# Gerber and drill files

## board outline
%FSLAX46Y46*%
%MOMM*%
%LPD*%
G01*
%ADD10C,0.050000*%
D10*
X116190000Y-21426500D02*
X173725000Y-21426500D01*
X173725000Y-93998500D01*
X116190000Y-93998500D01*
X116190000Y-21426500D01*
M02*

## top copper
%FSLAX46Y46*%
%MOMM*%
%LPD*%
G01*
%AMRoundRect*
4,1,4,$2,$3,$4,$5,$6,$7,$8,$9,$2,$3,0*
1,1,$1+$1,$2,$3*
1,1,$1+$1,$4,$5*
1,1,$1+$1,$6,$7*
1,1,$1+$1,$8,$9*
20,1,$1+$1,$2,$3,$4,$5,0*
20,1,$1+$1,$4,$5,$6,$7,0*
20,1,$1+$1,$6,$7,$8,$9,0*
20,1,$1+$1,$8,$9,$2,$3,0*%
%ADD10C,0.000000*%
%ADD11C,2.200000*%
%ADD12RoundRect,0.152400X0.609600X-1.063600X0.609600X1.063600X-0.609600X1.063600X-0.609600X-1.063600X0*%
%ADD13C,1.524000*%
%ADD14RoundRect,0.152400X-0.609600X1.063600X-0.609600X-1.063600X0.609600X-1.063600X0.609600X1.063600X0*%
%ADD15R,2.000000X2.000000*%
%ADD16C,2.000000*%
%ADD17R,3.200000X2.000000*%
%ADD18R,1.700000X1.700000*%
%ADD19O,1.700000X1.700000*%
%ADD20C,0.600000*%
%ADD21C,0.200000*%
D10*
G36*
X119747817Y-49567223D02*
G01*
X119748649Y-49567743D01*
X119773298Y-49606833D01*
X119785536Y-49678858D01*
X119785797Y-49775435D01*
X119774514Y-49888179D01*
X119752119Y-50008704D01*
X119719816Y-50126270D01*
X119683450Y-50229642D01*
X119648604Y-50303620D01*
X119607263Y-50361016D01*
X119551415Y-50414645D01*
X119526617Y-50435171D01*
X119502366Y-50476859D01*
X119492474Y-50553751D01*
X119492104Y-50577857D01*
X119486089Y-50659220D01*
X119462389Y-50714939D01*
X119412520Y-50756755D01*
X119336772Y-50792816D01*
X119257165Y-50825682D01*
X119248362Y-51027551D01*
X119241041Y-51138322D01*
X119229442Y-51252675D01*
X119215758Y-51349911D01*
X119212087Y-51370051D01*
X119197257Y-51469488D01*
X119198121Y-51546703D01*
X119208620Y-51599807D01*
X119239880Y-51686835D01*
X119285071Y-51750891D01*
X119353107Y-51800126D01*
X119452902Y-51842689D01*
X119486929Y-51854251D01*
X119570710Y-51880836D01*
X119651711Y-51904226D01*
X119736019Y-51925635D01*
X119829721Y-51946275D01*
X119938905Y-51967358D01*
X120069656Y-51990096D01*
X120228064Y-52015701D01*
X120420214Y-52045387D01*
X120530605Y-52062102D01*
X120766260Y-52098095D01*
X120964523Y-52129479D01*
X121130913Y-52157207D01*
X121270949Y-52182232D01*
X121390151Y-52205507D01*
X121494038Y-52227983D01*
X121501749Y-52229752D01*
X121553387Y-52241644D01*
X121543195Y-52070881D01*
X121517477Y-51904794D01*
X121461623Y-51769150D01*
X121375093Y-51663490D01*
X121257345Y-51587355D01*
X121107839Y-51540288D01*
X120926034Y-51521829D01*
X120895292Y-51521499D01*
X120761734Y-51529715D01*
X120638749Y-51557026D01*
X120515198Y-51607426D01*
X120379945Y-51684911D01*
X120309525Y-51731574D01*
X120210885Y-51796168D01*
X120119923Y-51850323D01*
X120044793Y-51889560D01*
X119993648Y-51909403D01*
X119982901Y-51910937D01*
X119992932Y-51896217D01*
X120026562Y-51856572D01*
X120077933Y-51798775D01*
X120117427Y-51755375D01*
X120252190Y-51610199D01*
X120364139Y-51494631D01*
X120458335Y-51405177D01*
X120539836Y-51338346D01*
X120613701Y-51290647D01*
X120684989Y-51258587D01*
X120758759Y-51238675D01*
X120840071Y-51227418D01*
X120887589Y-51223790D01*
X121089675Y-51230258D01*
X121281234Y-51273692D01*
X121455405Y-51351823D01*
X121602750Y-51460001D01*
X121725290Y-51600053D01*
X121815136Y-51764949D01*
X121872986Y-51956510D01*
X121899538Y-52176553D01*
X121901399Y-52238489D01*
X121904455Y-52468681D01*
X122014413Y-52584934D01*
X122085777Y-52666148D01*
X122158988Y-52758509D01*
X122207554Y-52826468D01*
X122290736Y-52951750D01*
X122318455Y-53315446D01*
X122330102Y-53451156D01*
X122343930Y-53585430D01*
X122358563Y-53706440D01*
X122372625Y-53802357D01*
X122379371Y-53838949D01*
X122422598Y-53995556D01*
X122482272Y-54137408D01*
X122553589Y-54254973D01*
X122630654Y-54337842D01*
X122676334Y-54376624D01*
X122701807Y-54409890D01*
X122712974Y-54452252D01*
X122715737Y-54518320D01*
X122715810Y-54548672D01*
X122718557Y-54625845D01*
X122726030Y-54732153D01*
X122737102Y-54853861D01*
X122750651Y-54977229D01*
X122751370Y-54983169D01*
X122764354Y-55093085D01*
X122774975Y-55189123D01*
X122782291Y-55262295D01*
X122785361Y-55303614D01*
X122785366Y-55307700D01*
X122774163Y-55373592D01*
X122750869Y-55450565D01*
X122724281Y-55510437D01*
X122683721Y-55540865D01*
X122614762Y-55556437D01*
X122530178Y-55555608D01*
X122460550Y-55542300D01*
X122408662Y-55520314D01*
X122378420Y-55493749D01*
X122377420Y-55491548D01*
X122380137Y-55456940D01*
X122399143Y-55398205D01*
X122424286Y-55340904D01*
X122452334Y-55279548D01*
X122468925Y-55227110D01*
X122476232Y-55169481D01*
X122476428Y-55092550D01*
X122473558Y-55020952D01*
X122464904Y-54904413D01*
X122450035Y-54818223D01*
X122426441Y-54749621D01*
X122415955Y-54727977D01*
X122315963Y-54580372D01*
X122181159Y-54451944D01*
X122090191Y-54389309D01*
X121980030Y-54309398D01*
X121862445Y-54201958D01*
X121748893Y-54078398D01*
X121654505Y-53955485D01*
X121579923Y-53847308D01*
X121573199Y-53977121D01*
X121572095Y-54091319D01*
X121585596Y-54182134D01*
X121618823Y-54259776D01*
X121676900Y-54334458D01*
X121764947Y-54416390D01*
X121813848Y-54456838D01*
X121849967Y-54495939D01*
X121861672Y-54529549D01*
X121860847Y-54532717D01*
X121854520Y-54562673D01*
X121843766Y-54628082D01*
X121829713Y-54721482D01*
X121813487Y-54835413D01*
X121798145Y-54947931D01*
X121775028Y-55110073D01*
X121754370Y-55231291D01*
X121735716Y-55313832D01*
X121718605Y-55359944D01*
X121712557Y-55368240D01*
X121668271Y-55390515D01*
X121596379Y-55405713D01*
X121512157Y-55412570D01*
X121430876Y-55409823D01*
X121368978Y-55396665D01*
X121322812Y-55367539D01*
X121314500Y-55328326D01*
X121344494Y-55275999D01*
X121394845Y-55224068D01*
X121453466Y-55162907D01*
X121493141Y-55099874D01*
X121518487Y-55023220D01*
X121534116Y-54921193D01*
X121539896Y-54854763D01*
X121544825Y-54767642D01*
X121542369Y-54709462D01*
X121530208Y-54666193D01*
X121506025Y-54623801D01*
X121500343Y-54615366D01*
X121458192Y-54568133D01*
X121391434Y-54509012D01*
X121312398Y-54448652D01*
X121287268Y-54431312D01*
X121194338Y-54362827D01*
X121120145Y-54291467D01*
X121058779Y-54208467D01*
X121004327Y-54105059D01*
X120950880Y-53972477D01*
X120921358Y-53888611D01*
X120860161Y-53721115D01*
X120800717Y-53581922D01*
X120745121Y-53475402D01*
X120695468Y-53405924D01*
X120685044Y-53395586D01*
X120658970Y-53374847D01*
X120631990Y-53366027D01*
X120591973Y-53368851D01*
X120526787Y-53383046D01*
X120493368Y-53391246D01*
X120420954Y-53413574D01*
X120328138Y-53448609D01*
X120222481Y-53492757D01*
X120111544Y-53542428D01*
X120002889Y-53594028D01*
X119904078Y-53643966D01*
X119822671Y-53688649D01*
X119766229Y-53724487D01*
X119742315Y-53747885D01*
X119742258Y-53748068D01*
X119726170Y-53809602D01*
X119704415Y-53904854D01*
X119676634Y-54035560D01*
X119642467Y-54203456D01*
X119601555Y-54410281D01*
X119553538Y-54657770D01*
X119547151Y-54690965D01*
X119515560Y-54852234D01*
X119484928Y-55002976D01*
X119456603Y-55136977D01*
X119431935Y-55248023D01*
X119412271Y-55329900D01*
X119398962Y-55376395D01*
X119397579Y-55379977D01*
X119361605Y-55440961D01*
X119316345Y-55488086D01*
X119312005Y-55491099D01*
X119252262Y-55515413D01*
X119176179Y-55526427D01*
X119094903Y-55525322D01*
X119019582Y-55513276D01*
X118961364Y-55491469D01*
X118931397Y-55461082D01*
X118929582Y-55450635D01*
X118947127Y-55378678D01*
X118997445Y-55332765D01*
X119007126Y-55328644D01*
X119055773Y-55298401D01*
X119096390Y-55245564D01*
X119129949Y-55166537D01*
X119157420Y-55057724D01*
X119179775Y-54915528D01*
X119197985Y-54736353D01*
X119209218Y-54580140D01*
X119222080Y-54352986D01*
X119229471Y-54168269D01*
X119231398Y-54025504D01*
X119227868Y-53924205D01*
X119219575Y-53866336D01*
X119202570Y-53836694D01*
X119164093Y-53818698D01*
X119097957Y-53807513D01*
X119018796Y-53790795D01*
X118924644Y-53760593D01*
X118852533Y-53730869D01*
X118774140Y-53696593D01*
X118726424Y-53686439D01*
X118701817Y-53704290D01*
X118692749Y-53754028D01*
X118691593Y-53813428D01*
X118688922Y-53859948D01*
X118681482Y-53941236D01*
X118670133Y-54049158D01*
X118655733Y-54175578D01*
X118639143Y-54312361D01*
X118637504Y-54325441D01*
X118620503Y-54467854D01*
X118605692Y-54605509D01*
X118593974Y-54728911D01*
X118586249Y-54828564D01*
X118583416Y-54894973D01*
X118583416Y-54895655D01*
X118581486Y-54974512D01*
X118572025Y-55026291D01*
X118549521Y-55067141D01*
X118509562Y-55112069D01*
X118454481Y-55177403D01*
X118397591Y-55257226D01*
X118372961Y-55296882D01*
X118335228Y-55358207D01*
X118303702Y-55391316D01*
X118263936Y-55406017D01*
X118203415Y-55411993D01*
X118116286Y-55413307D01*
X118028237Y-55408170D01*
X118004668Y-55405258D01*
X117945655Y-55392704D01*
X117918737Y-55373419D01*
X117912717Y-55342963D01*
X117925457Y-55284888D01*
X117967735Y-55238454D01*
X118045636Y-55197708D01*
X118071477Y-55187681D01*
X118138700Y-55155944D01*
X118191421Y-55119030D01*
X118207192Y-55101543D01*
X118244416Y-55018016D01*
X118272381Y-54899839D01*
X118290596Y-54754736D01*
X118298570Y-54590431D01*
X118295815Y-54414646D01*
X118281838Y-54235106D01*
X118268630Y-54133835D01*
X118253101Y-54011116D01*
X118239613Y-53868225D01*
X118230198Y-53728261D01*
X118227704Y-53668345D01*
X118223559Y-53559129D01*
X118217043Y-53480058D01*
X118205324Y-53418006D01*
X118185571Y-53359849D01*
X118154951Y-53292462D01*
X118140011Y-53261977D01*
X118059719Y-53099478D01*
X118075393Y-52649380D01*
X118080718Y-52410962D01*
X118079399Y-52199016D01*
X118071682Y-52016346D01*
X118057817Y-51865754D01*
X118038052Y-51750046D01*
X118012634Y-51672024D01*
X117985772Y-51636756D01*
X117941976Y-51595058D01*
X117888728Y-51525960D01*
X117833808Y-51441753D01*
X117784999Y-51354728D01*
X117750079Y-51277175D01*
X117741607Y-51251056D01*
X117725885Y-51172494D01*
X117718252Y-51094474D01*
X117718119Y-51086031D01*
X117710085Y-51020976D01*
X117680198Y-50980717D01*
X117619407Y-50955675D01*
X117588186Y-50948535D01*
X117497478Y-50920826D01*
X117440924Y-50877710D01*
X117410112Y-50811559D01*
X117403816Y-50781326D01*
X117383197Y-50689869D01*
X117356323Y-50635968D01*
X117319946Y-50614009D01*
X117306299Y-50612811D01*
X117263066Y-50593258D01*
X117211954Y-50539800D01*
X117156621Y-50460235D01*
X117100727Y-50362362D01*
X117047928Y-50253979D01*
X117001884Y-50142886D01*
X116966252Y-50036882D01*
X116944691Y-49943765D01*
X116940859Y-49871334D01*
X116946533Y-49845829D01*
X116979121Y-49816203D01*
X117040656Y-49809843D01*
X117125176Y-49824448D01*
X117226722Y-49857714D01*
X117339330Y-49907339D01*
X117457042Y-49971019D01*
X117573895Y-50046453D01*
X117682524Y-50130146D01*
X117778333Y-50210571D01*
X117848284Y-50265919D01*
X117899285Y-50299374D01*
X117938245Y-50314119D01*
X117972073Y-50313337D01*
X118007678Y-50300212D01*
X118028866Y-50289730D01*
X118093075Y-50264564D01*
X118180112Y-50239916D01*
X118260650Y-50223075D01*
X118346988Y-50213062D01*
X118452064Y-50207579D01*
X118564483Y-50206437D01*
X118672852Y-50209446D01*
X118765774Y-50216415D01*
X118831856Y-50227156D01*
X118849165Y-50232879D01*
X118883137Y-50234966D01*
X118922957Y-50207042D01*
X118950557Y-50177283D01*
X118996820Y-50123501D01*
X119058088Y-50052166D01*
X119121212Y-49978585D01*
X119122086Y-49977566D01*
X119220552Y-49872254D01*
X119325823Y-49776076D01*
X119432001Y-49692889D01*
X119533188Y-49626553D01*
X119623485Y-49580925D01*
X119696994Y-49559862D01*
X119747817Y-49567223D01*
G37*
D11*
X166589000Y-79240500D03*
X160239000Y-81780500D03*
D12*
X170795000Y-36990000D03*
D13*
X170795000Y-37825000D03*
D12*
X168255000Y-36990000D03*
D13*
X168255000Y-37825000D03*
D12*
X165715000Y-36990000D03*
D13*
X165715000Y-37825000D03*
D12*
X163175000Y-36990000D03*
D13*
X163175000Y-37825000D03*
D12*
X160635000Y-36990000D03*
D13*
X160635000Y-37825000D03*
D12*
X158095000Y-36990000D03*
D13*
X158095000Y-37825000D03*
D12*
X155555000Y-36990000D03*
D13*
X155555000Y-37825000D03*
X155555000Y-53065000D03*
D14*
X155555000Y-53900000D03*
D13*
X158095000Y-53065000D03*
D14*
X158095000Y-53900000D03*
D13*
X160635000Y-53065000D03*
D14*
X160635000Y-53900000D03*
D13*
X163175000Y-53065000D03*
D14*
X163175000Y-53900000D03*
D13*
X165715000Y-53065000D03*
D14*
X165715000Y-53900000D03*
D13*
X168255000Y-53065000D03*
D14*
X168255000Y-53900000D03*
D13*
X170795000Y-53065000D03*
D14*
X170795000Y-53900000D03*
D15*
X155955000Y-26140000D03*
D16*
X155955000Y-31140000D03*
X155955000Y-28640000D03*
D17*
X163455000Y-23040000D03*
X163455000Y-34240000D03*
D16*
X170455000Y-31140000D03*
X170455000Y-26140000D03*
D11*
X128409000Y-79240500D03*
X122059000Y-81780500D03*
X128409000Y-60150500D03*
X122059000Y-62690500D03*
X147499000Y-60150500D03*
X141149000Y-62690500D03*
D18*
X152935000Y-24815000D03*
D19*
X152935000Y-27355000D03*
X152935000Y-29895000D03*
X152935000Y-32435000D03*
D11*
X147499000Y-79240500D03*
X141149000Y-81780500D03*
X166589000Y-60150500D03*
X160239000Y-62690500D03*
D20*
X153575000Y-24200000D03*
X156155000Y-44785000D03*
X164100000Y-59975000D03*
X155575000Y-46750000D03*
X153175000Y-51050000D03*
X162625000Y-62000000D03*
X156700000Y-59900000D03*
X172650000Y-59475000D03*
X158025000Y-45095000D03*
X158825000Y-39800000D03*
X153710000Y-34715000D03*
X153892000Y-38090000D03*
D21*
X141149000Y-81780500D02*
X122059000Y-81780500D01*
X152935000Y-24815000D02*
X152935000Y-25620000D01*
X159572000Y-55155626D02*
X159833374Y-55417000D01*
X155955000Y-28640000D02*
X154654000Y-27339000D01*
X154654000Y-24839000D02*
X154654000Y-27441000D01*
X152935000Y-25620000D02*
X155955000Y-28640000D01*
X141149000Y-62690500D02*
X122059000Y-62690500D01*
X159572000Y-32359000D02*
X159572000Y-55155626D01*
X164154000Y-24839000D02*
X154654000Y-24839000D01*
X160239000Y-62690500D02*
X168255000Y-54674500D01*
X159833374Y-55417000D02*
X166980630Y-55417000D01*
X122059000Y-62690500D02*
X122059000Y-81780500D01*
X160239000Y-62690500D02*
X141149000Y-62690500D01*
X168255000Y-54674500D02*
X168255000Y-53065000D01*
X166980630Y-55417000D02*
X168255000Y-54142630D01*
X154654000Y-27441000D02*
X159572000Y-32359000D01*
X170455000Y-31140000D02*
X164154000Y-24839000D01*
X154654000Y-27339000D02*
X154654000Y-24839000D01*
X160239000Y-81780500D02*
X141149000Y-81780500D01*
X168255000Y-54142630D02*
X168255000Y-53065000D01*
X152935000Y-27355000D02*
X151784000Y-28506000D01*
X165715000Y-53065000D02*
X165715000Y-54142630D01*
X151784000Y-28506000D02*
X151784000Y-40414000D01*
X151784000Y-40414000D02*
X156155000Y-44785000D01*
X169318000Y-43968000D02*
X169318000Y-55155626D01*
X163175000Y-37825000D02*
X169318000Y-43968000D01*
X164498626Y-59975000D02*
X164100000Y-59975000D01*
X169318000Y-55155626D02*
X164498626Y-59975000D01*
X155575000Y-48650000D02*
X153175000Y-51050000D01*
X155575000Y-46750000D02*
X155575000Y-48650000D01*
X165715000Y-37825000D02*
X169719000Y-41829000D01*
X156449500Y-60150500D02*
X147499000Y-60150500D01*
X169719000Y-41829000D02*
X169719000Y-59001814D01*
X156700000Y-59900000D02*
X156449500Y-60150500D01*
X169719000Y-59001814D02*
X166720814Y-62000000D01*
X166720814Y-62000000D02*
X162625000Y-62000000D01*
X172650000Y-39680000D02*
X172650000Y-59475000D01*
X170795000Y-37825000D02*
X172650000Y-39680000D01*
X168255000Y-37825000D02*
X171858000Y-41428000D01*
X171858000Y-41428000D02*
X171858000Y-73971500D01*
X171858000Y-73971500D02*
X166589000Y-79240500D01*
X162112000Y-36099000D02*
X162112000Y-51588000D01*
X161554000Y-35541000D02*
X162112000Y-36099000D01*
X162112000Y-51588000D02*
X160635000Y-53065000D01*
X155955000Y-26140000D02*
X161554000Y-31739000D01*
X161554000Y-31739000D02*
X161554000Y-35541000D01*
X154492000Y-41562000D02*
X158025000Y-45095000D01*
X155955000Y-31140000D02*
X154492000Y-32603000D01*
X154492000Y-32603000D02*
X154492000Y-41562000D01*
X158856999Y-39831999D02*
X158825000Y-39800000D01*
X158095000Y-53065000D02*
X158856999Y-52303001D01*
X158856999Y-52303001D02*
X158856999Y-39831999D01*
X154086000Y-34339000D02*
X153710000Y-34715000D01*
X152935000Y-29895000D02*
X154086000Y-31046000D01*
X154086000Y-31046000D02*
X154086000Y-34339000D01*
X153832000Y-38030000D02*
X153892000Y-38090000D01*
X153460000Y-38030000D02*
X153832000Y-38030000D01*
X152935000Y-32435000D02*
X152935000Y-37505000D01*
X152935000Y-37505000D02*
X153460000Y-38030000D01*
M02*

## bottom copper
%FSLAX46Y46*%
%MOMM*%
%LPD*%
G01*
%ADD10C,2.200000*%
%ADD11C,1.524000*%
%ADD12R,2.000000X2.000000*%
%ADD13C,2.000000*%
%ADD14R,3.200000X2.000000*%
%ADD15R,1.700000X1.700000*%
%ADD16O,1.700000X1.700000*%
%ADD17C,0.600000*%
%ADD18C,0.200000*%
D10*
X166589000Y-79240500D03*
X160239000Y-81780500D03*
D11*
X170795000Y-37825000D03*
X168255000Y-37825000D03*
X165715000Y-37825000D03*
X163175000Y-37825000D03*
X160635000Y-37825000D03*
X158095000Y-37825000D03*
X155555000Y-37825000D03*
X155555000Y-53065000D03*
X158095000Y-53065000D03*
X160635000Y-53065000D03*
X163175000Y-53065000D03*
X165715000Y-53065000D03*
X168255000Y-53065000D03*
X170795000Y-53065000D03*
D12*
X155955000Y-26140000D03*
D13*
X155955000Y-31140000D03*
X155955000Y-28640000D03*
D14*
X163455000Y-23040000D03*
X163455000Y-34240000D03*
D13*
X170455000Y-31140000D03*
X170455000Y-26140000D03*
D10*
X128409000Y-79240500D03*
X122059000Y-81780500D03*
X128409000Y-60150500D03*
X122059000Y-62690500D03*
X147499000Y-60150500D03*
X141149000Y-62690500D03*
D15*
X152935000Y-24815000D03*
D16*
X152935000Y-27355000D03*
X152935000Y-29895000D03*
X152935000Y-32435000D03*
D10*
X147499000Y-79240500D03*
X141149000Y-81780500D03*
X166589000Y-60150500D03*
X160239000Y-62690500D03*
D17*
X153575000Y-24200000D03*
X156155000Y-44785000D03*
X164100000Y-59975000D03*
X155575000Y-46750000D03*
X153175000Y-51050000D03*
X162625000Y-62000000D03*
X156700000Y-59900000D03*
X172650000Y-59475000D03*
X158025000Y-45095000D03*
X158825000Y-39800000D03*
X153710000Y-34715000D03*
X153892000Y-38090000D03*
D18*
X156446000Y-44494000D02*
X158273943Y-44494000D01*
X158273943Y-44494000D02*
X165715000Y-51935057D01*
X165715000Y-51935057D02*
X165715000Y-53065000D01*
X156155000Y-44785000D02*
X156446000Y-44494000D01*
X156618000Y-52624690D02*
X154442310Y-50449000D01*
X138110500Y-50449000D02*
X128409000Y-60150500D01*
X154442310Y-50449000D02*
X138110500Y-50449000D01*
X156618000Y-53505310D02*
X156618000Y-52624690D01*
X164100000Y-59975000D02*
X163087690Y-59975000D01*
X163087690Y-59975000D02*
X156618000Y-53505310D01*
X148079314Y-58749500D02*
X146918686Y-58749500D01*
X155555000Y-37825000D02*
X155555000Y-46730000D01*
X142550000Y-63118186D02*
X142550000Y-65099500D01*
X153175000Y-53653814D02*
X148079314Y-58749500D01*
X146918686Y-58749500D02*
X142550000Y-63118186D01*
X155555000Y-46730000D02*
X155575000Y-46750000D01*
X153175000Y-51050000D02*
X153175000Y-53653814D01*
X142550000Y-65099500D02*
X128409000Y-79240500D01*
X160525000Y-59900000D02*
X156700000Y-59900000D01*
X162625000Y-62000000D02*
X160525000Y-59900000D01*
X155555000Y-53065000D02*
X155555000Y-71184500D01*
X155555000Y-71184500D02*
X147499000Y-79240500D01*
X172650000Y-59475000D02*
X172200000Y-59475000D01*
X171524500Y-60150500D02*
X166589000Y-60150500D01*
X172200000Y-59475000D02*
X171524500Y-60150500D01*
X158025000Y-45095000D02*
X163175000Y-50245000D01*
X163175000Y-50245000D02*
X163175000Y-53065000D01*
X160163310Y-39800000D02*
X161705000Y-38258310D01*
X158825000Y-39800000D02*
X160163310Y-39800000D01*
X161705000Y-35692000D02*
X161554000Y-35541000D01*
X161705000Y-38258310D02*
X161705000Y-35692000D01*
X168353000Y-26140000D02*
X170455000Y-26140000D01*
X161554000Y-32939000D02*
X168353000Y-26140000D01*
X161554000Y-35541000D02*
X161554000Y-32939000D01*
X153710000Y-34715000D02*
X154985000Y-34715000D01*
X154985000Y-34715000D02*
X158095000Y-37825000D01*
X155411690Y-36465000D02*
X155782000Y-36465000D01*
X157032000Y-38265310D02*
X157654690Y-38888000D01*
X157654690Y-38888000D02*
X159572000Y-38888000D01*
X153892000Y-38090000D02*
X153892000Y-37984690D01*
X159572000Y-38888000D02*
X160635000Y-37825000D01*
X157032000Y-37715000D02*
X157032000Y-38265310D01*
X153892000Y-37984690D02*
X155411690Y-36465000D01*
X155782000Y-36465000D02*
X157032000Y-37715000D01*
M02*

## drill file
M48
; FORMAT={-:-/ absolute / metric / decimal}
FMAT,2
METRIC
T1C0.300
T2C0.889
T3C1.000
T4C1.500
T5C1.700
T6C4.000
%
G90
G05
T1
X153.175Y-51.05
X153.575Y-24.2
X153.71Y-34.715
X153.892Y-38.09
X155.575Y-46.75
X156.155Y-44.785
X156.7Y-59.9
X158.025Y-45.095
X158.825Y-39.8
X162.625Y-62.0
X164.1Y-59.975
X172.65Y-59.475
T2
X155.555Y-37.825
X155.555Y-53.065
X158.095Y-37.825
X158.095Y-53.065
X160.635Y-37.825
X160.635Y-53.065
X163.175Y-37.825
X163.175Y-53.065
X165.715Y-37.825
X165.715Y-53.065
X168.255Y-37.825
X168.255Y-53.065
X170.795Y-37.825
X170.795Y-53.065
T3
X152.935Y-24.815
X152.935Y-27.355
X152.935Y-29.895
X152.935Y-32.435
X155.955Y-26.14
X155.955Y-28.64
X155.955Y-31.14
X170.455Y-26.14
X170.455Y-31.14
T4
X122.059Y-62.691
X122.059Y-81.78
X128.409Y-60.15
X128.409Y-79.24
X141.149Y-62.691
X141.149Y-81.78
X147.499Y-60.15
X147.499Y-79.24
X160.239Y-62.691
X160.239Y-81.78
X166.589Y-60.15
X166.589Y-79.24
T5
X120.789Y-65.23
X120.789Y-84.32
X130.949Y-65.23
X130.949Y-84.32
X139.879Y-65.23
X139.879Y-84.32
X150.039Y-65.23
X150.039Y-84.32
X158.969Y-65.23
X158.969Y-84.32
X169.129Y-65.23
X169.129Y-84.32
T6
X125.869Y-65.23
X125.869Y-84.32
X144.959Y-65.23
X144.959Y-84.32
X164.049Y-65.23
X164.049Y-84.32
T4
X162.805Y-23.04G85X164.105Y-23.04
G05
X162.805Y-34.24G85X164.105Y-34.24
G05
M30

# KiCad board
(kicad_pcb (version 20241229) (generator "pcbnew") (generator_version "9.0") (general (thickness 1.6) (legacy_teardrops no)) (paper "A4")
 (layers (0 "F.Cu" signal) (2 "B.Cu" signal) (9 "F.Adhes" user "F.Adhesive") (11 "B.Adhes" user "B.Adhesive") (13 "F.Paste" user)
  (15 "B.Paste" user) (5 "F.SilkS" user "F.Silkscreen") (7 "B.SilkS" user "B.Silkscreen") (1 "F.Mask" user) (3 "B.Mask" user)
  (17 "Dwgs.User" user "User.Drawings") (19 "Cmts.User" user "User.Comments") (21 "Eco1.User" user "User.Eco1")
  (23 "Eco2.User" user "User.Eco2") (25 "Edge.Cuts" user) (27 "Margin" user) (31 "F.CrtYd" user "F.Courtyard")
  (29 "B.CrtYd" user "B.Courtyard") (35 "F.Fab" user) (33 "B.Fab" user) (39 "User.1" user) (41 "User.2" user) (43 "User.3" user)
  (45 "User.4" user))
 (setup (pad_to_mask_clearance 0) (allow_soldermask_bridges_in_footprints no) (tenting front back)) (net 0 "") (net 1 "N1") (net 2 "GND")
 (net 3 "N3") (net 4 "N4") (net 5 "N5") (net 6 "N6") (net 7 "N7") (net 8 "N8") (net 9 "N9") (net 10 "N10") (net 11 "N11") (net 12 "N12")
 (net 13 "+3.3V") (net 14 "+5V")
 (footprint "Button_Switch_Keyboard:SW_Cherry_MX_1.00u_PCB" (layer "F.Cu") (at 166.589 79.2405)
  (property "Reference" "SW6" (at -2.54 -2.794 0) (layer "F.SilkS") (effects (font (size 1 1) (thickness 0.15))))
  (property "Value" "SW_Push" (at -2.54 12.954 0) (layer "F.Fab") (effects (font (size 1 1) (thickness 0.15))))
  (pad "" np_thru_hole circle (at -7.62 5.08) (size 1.7 1.7) (drill 1.7) (layers "*.Cu" "*.Mask"))
  (pad "" np_thru_hole circle (at -2.54 5.08) (size 4 4) (drill 4) (layers "*.Cu" "*.Mask"))
  (pad "" np_thru_hole circle (at 2.54 5.08) (size 1.7 1.7) (drill 1.7) (layers "*.Cu" "*.Mask"))
  (pad "1" thru_hole circle (at 0 0) (size 2.2 2.2) (drill 1.5) (layers "*.Cu" "*.Mask") (remove_unused_layers no) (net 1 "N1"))
  (pad "2" thru_hole circle (at -6.35 2.54) (size 2.2 2.2) (drill 1.5) (layers "*.Cu" "*.Mask") (remove_unused_layers no) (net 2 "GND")))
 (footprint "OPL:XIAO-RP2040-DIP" (layer "F.Cu") (at 163.175 45.445 -90)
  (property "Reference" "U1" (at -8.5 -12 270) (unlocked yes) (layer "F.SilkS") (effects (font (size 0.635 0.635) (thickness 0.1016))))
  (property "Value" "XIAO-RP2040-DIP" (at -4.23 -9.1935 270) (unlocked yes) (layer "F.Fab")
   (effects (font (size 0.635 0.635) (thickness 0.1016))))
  (pad "1" smd roundrect (at -8.455 -7.62 90) (size 2.432 1.524) (layers "F.Cu" "F.Mask") (roundrect_rratio 0.1) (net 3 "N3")
   (thermal_bridge_angle 45))
  (pad "1" thru_hole circle (at -7.62 -7.62 90) (size 1.524 1.524) (drill 0.889) (layers "*.Cu" "*.Mask") (remove_unused_layers no)
   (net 3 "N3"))
  (pad "2" smd roundrect (at -8.455 -5.08 90) (size 2.432 1.524) (layers "F.Cu" "F.Mask") (roundrect_rratio 0.1) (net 1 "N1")
   (thermal_bridge_angle 45))
  (pad "2" thru_hole circle (at -7.62 -5.08 90) (size 1.524 1.524) (drill 0.889) (layers "*.Cu" "*.Mask") (remove_unused_layers no)
   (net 1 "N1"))
  (pad "3" smd roundrect (at -8.455 -2.54 90) (size 2.432 1.524) (layers "F.Cu" "F.Mask") (roundrect_rratio 0.1) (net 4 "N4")
   (thermal_bridge_angle 45))
  (pad "3" thru_hole circle (at -7.62 -2.54 90) (size 1.524 1.524) (drill 0.889) (layers "*.Cu" "*.Mask") (remove_unused_layers no)
   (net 4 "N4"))
  (pad "4" smd roundrect (at -8.455 0 90) (size 2.432 1.524) (layers "F.Cu" "F.Mask") (roundrect_rratio 0.1) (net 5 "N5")
   (thermal_bridge_angle 45))
  (pad "4" thru_hole circle (at -7.62 0 90) (size 1.524 1.524) (drill 0.889) (layers "*.Cu" "*.Mask") (remove_unused_layers no) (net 5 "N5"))
  (pad "5" smd roundrect (at -8.455 2.54 90) (size 2.432 1.524) (layers "F.Cu" "F.Mask") (roundrect_rratio 0.1) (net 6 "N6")
   (thermal_bridge_angle 45))
  (pad "5" thru_hole circle (at -7.62 2.54 90) (size 1.524 1.524) (drill 0.889) (layers "*.Cu" "*.Mask") (remove_unused_layers no)
   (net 6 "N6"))
  (pad "6" smd roundrect (at -8.455 5.08 90) (size 2.432 1.524) (layers "F.Cu" "F.Mask") (roundrect_rratio 0.1) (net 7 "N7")
   (thermal_bridge_angle 45))
  (pad "6" thru_hole circle (at -7.62 5.08 90) (size 1.524 1.524) (drill 0.889) (layers "*.Cu" "*.Mask") (remove_unused_layers no)
   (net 7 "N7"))
  (pad "7" smd roundrect (at -8.455 7.62 90) (size 2.432 1.524) (layers "F.Cu" "F.Mask") (roundrect_rratio 0.1) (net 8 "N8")
   (thermal_bridge_angle 45))
  (pad "7" thru_hole circle (at -7.62 7.62 90) (size 1.524 1.524) (drill 0.889) (layers "*.Cu" "*.Mask") (remove_unused_layers no)
   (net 8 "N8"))
  (pad "8" thru_hole circle (at 7.62 7.62 270) (size 1.524 1.524) (drill 0.889) (layers "*.Cu" "*.Mask") (remove_unused_layers no)
   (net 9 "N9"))
  (pad "8" smd roundrect (at 8.455 7.62 270) (size 2.432 1.524) (layers "F.Cu" "F.Mask") (roundrect_rratio 0.1) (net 9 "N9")
   (thermal_bridge_angle 45))
  (pad "9" thru_hole circle (at 7.62 5.08 270) (size 1.524 1.524) (drill 0.889) (layers "*.Cu" "*.Mask") (remove_unused_layers no)
   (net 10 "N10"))
  (pad "9" smd roundrect (at 8.455 5.08 270) (size 2.432 1.524) (layers "F.Cu" "F.Mask") (roundrect_rratio 0.1) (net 10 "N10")
   (thermal_bridge_angle 45))
  (pad "10" thru_hole circle (at 7.62 2.54 270) (size 1.524 1.524) (drill 0.889) (layers "*.Cu" "*.Mask") (remove_unused_layers no)
   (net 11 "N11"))
  (pad "10" smd roundrect (at 8.455 2.54 270) (size 2.432 1.524) (layers "F.Cu" "F.Mask") (roundrect_rratio 0.1) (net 11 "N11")
   (thermal_bridge_angle 45))
  (pad "11" thru_hole circle (at 7.62 0 270) (size 1.524 1.524) (drill 0.889) (layers "*.Cu" "*.Mask") (remove_unused_layers no)
   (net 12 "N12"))
  (pad "11" smd roundrect (at 8.455 0 270) (size 2.432 1.524) (layers "F.Cu" "F.Mask") (roundrect_rratio 0.1) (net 12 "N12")
   (thermal_bridge_angle 45))
  (pad "12" thru_hole circle (at 7.62 -2.54 270) (size 1.524 1.524) (drill 0.889) (layers "*.Cu" "*.Mask") (remove_unused_layers no)
   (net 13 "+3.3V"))
  (pad "12" smd roundrect (at 8.455 -2.54 270) (size 2.432 1.524) (layers "F.Cu" "F.Mask") (roundrect_rratio 0.1) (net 13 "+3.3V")
   (thermal_bridge_angle 45))
  (pad "13" thru_hole circle (at 7.62 -5.08 270) (size 1.524 1.524) (drill 0.889) (layers "*.Cu" "*.Mask") (remove_unused_layers no)
   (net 2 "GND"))
  (pad "13" smd roundrect (at 8.455 -5.08 270) (size 2.432 1.524) (layers "F.Cu" "F.Mask") (roundrect_rratio 0.1) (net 2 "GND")
   (thermal_bridge_angle 45))
  (pad "14" thru_hole circle (at 7.62 -7.62 270) (size 1.524 1.524) (drill 0.889) (layers "*.Cu" "*.Mask") (remove_unused_layers no)
   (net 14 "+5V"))
  (pad "14" smd roundrect (at 8.455 -7.62 270) (size 2.432 1.524) (layers "F.Cu" "F.Mask") (roundrect_rratio 0.1) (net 14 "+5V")
   (thermal_bridge_angle 45)))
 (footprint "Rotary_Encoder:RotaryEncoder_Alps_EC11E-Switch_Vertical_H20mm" (layer "F.Cu") (at 155.955 26.14)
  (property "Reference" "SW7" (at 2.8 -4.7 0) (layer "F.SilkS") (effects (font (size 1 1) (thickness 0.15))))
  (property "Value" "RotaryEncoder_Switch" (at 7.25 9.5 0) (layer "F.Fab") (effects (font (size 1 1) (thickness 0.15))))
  (pad "A" thru_hole rect (at 0 0) (size 2 2) (drill 1) (layers "*.Cu" "*.Mask") (remove_unused_layers no) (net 11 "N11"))
  (pad "B" thru_hole circle (at 0 5) (size 2 2) (drill 1) (layers "*.Cu" "*.Mask") (remove_unused_layers no) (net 12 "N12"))
  (pad "C" thru_hole circle (at 0 2.5) (size 2 2) (drill 1) (layers "*.Cu" "*.Mask") (remove_unused_layers no) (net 2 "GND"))
  (pad "MP" thru_hole rect (at 7.5 -3.1) (size 3.2 2) (drill oval 2.8 1.5) (layers "*.Cu" "*.Mask") (remove_unused_layers no))
  (pad "MP" thru_hole rect (at 7.5 8.1) (size 3.2 2) (drill oval 2.8 1.5) (layers "*.Cu" "*.Mask") (remove_unused_layers no))
  (pad "S1" thru_hole circle (at 14.5 5) (size 2 2) (drill 1) (layers "*.Cu" "*.Mask") (remove_unused_layers no) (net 2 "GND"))
  (pad "S2" thru_hole circle (at 14.5 0) (size 2 2) (drill 1) (layers "*.Cu" "*.Mask") (remove_unused_layers no) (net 10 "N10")))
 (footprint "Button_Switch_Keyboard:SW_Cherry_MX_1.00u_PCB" (layer "F.Cu") (at 128.409 79.2405)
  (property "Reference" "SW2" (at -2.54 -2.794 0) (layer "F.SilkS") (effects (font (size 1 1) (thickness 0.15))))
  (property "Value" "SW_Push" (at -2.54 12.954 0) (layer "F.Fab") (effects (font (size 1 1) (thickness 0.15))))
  (pad "" np_thru_hole circle (at -7.62 5.08) (size 1.7 1.7) (drill 1.7) (layers "*.Cu" "*.Mask"))
  (pad "" np_thru_hole circle (at -2.54 5.08) (size 4 4) (drill 4) (layers "*.Cu" "*.Mask"))
  (pad "" np_thru_hole circle (at 2.54 5.08) (size 1.7 1.7) (drill 1.7) (layers "*.Cu" "*.Mask"))
  (pad "1" thru_hole circle (at 0 0) (size 2.2 2.2) (drill 1.5) (layers "*.Cu" "*.Mask") (remove_unused_layers no) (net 8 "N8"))
  (pad "2" thru_hole circle (at -6.35 2.54) (size 2.2 2.2) (drill 1.5) (layers "*.Cu" "*.Mask") (remove_unused_layers no) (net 2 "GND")))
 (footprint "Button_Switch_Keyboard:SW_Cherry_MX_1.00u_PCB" (layer "F.Cu") (at 128.409 60.1505)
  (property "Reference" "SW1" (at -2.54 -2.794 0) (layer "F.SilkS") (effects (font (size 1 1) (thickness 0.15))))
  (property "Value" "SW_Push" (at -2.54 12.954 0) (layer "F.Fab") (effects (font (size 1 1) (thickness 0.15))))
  (pad "" np_thru_hole circle (at -7.62 5.08) (size 1.7 1.7) (drill 1.7) (layers "*.Cu" "*.Mask"))
  (pad "" np_thru_hole circle (at -2.54 5.08) (size 4 4) (drill 4) (layers "*.Cu" "*.Mask"))
  (pad "" np_thru_hole circle (at 2.54 5.08) (size 1.7 1.7) (drill 1.7) (layers "*.Cu" "*.Mask"))
  (pad "1" thru_hole circle (at 0 0) (size 2.2 2.2) (drill 1.5) (layers "*.Cu" "*.Mask") (remove_unused_layers no) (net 5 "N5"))
  (pad "2" thru_hole circle (at -6.35 2.54) (size 2.2 2.2) (drill 1.5) (layers "*.Cu" "*.Mask") (remove_unused_layers no) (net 2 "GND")))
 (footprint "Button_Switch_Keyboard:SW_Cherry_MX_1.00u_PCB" (layer "F.Cu") (at 147.499 60.1505)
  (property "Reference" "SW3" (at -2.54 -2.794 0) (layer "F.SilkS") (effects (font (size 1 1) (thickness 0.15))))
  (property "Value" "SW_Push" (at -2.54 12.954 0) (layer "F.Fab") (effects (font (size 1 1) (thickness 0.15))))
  (pad "" np_thru_hole circle (at -7.62 5.08) (size 1.7 1.7) (drill 1.7) (layers "*.Cu" "*.Mask"))
  (pad "" np_thru_hole circle (at -2.54 5.08) (size 4 4) (drill 4) (layers "*.Cu" "*.Mask"))
  (pad "" np_thru_hole circle (at 2.54 5.08) (size 1.7 1.7) (drill 1.7) (layers "*.Cu" "*.Mask"))
  (pad "1" thru_hole circle (at 0 0) (size 2.2 2.2) (drill 1.5) (layers "*.Cu" "*.Mask") (remove_unused_layers no) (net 4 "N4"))
  (pad "2" thru_hole circle (at -6.35 2.54) (size 2.2 2.2) (drill 1.5) (layers "*.Cu" "*.Mask") (remove_unused_layers no) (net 2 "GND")))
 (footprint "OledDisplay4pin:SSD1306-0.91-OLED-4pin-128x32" (layer "F.Cu") (at 116.435 22.625)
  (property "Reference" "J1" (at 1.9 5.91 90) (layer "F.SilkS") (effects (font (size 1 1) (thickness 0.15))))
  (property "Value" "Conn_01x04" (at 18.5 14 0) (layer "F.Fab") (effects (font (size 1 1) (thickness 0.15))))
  (pad "1" thru_hole rect (at 36.5 2.19) (size 1.7 1.7) (drill 1) (layers "*.Cu" "*.Mask") (remove_unused_layers no) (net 2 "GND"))
  (pad "2" thru_hole oval (at 36.5 4.73) (size 1.7 1.7) (drill 1) (layers "*.Cu" "*.Mask") (remove_unused_layers no) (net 13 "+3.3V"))
  (pad "3" thru_hole oval (at 36.5 7.27) (size 1.7 1.7) (drill 1) (layers "*.Cu" "*.Mask") (remove_unused_layers no) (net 7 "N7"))
  (pad "4" thru_hole oval (at 36.5 9.81) (size 1.7 1.7) (drill 1) (layers "*.Cu" "*.Mask") (remove_unused_layers no) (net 6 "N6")))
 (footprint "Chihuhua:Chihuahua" (layer "F.Cu") (at 119.795 52.56)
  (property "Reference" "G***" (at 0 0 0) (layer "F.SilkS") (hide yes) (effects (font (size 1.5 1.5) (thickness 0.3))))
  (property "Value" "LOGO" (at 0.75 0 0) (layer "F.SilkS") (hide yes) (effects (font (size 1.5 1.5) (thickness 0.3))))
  (fp_poly
   (pts (xy -0.047183 -2.992777) (xy -0.046351 -2.992257) (xy -0.021702 -2.953167) (xy -0.009464 -2.881142) (xy -0.009203 -2.784565)
    (xy -0.020486 -2.671821) (xy -0.042881 -2.551296) (xy -0.075184 -2.43373) (xy -0.11155 -2.330358) (xy -0.146396 -2.25638)
    (xy -0.187737 -2.198984) (xy -0.243585 -2.145355) (xy -0.268383 -2.124829) (xy -0.292634 -2.083141) (xy -0.302526 -2.006249)
    (xy -0.302896 -1.982143) (xy -0.308911 -1.90078) (xy -0.332611 -1.845061) (xy -0.38248 -1.803245) (xy -0.458228 -1.767184)
    (xy -0.537835 -1.734318) (xy -0.546638 -1.532449) (xy -0.553959 -1.421678) (xy -0.565558 -1.307325) (xy -0.579242 -1.210089)
    (xy -0.582913 -1.189949) (xy -0.597743 -1.090512) (xy -0.596879 -1.013297) (xy -0.58638 -0.960193) (xy -0.55512 -0.873165)
    (xy -0.509929 -0.809109) (xy -0.441893 -0.759874) (xy -0.342098 -0.717311) (xy -0.308071 -0.705749) (xy -0.22429 -0.679164)
    (xy -0.143289 -0.655774) (xy -0.058981 -0.634365) (xy 0.034721 -0.613725) (xy 0.143905 -0.592642) (xy 0.274656 -0.569904)
    (xy 0.433064 -0.544299) (xy 0.625214 -0.514613) (xy 0.735605 -0.497898) (xy 0.97126 -0.461905) (xy 1.169523 -0.430521)
    (xy 1.335913 -0.402793) (xy 1.475949 -0.377768) (xy 1.595151 -0.354493) (xy 1.699038 -0.332017) (xy 1.706749 -0.330248)
    (xy 1.758387 -0.318356) (xy 1.748195 -0.489119) (xy 1.722477 -0.655206) (xy 1.666623 -0.79085) (xy 1.580093 -0.89651)
    (xy 1.462345 -0.972645) (xy 1.312839 -1.019712) (xy 1.131034 -1.038171) (xy 1.100292 -1.038501) (xy 0.966734 -1.030285)
    (xy 0.843749 -1.002974) (xy 0.720198 -0.952574) (xy 0.584945 -0.875089) (xy 0.514525 -0.828426) (xy 0.415885 -0.763832)
    (xy 0.324923 -0.709677) (xy 0.249793 -0.67044) (xy 0.198648 -0.650597) (xy 0.187901 -0.649063) (xy 0.197932 -0.663783)
    (xy 0.231562 -0.703428) (xy 0.282933 -0.761225) (xy 0.322427 -0.804625) (xy 0.45719 -0.949801) (xy 0.569139 -1.065369)
    (xy 0.663335 -1.154823) (xy 0.744836 -1.221654) (xy 0.818701 -1.269353) (xy 0.889989 -1.301413) (xy 0.963759 -1.321325)
    (xy 1.045071 -1.332582) (xy 1.092589 -1.33621) (xy 1.294675 -1.329742) (xy 1.486234 -1.286308) (xy 1.660405 -1.208177)
    (xy 1.80775 -1.099999) (xy 1.93029 -0.959947) (xy 2.020136 -0.795051) (xy 2.077986 -0.60349) (xy 2.104538 -0.383447)
    (xy 2.106399 -0.321511) (xy 2.109455 -0.091319) (xy 2.219413 0.024934) (xy 2.290777 0.106148) (xy 2.363988 0.198509)
    (xy 2.412554 0.266468) (xy 2.495736 0.39175) (xy 2.523455 0.755446) (xy 2.535102 0.891156) (xy 2.54893 1.02543) (xy 2.563563 1.14644)
    (xy 2.577625 1.242357) (xy 2.584371 1.278949) (xy 2.627598 1.435556) (xy 2.687272 1.577408) (xy 2.758589 1.694973)
    (xy 2.835654 1.777842) (xy 2.881334 1.816624) (xy 2.906807 1.84989) (xy 2.917974 1.892252) (xy 2.920737 1.95832) (xy 2.92081 1.988672)
    (xy 2.923557 2.065845) (xy 2.93103 2.172153) (xy 2.942102 2.293861) (xy 2.955651 2.417229) (xy 2.95637 2.423169) (xy 2.969354 2.533085)
    (xy 2.979975 2.629123) (xy 2.987291 2.702295) (xy 2.990361 2.743614) (xy 2.990366 2.7477) (xy 2.979163 2.813592) (xy 2.955869 2.890565)
    (xy 2.929281 2.950437) (xy 2.888721 2.980865) (xy 2.819762 2.996437) (xy 2.735178 2.995608) (xy 2.66555 2.9823) (xy 2.613662 2.960314)
    (xy 2.58342 2.933749) (xy 2.58242 2.931548) (xy 2.585137 2.89694) (xy 2.604143 2.838205) (xy 2.629286 2.780904) (xy 2.657334 2.719548)
    (xy 2.673925 2.66711) (xy 2.681232 2.609481) (xy 2.681428 2.53255) (xy 2.678558 2.460952) (xy 2.669904 2.344413) (xy 2.655035 2.258223)
    (xy 2.631441 2.189621) (xy 2.620955 2.167977) (xy 2.520963 2.020372) (xy 2.386159 1.891944) (xy 2.295191 1.829309) (xy 2.18503 1.749398)
    (xy 2.067445 1.641958) (xy 1.953893 1.518398) (xy 1.859505 1.395485) (xy 1.784923 1.287308) (xy 1.778199 1.417121)
    (xy 1.777095 1.531319) (xy 1.790596 1.622134) (xy 1.823823 1.699776) (xy 1.8819 1.774458) (xy 1.969947 1.85639) (xy 2.018848 1.896838)
    (xy 2.054967 1.935939) (xy 2.066672 1.969549) (xy 2.065847 1.972717) (xy 2.05952 2.002673) (xy 2.048766 2.068082) (xy 2.034713 2.161482)
    (xy 2.018487 2.275413) (xy 2.003145 2.387931) (xy 1.980028 2.550073) (xy 1.95937 2.671291) (xy 1.940716 2.753832) (xy 1.923605 2.799944)
    (xy 1.917557 2.80824) (xy 1.873271 2.830515) (xy 1.801379 2.845713) (xy 1.717157 2.85257) (xy 1.635876 2.849823) (xy 1.573978 2.836665)
    (xy 1.527812 2.807539) (xy 1.5195 2.768326) (xy 1.549494 2.715999) (xy 1.599845 2.664068) (xy 1.658466 2.602907) (xy 1.698141 2.539874)
    (xy 1.723487 2.46322) (xy 1.739116 2.361193) (xy 1.744896 2.294763) (xy 1.749825 2.207642) (xy 1.747369 2.149462) (xy 1.735208 2.106193)
    (xy 1.711025 2.063801) (xy 1.705343 2.055366) (xy 1.663192 2.008133) (xy 1.596434 1.949012) (xy 1.517398 1.888652)
    (xy 1.492268 1.871312) (xy 1.399338 1.802827) (xy 1.325145 1.731467) (xy 1.263779 1.648467) (xy 1.209327 1.545059) (xy 1.15588 1.412477)
    (xy 1.126358 1.328611) (xy 1.065161 1.161115) (xy 1.005717 1.021922) (xy 0.950121 0.915402) (xy 0.900468 0.845924)
    (xy 0.890044 0.835586) (xy 0.86397 0.814847) (xy 0.83699 0.806027) (xy 0.796973 0.808851) (xy 0.731787 0.823046) (xy 0.698368 0.831246)
    (xy 0.625954 0.853574) (xy 0.533138 0.888609) (xy 0.427481 0.932757) (xy 0.316544 0.982428) (xy 0.207889 1.034028)
    (xy 0.109078 1.083966) (xy 0.027671 1.128649) (xy -0.028771 1.164487) (xy -0.052685 1.187885) (xy -0.052742 1.188068)
    (xy -0.06883 1.249602) (xy -0.090585 1.344854) (xy -0.118366 1.47556) (xy -0.152533 1.643456) (xy -0.193445 1.850281)
    (xy -0.241462 2.09777) (xy -0.247849 2.130965) (xy -0.27944 2.292234) (xy -0.310072 2.442976) (xy -0.338397 2.576977)
    (xy -0.363065 2.688023) (xy -0.382729 2.7699) (xy -0.396038 2.816395) (xy -0.397421 2.819977) (xy -0.433395 2.880961)
    (xy -0.478655 2.928086) (xy -0.482995 2.931099) (xy -0.542738 2.955413) (xy -0.618821 2.966427) (xy -0.700097 2.965322)
    (xy -0.775418 2.953276) (xy -0.833636 2.931469) (xy -0.863603 2.901082) (xy -0.865418 2.890635) (xy -0.847873 2.818678)
    (xy -0.797555 2.772765) (xy -0.787874 2.768644) (xy -0.739227 2.738401) (xy -0.69861 2.685564) (xy -0.665051 2.606537)
    (xy -0.63758 2.497724) (xy -0.615225 2.355528) (xy -0.597015 2.176353) (xy -0.585782 2.02014) (xy -0.57292 1.792986)
    (xy -0.565529 1.608269) (xy -0.563602 1.465504) (xy -0.567132 1.364205) (xy -0.575425 1.306336) (xy -0.59243 1.276694)
    (xy -0.630907 1.258698) (xy -0.697043 1.247513) (xy -0.776204 1.230795) (xy -0.870356 1.200593) (xy -0.942467 1.170869)
    (xy -1.02086 1.136593) (xy -1.068576 1.126439) (xy -1.093183 1.14429) (xy -1.102251 1.194028) (xy -1.103407 1.253428)
    (xy -1.106078 1.299948) (xy -1.113518 1.381236) (xy -1.124867 1.489158) (xy -1.139267 1.615578) (xy -1.155857 1.752361)
    (xy -1.157496 1.765441) (xy -1.174497 1.907854) (xy -1.189308 2.045509) (xy -1.201026 2.168911) (xy -1.208751 2.268564)
    (xy -1.211584 2.334973) (xy -1.211584 2.335655) (xy -1.213514 2.414512) (xy -1.222975 2.466291) (xy -1.245479 2.507141)
    (xy -1.285438 2.552069) (xy -1.340519 2.617403) (xy -1.397409 2.697226) (xy -1.422039 2.736882) (xy -1.459772 2.798207)
    (xy -1.491298 2.831316) (xy -1.531064 2.846017) (xy -1.591585 2.851993) (xy -1.678714 2.853307) (xy -1.766763 2.84817)
    (xy -1.790332 2.845258) (xy -1.849345 2.832704) (xy -1.876263 2.813419) (xy -1.882283 2.782963) (xy -1.869543 2.724888)
    (xy -1.827265 2.678454) (xy -1.749364 2.637708) (xy -1.723523 2.627681) (xy -1.6563 2.595944) (xy -1.603579 2.55903)
    (xy -1.587808 2.541543) (xy -1.550584 2.458016) (xy -1.522619 2.339839) (xy -1.504404 2.194736) (xy -1.49643 2.030431)
    (xy -1.499185 1.854646) (xy -1.513162 1.675106) (xy -1.52637 1.573835) (xy -1.541899 1.451116) (xy -1.555387 1.308225)
    (xy -1.564802 1.168261) (xy -1.567296 1.108345) (xy -1.571441 0.999129) (xy -1.577957 0.920058) (xy -1.589676 0.858006)
    (xy -1.609429 0.799849) (xy -1.640049 0.732462) (xy -1.654989 0.701977) (xy -1.735281 0.539478) (xy -1.719607 0.08938)
    (xy -1.714282 -0.149038) (xy -1.715601 -0.360984) (xy -1.723318 -0.543654) (xy -1.737183 -0.694246) (xy -1.756948 -0.809954)
    (xy -1.782366 -0.887976) (xy -1.809228 -0.923244) (xy -1.853024 -0.964942) (xy -1.906272 -1.03404) (xy -1.961192 -1.118247)
    (xy -2.010001 -1.205272) (xy -2.044921 -1.282825) (xy -2.053393 -1.308944) (xy -2.069115 -1.387506) (xy -2.076748 -1.465526)
    (xy -2.076881 -1.473969) (xy -2.084915 -1.539024) (xy -2.114802 -1.579283) (xy -2.175593 -1.604325) (xy -2.206814 -1.611465)
    (xy -2.297522 -1.639174) (xy -2.354076 -1.68229) (xy -2.384888 -1.748441) (xy -2.391184 -1.778674) (xy -2.411803 -1.870131)
    (xy -2.438677 -1.924032) (xy -2.475054 -1.945991) (xy -2.488701 -1.947189) (xy -2.531934 -1.966742) (xy -2.583046 -2.0202)
    (xy -2.638379 -2.099765) (xy -2.694273 -2.197638) (xy -2.747072 -2.306021) (xy -2.793116 -2.417114) (xy -2.828748 -2.523118)
    (xy -2.850309 -2.616235) (xy -2.854141 -2.688666) (xy -2.848467 -2.714171) (xy -2.815879 -2.743797) (xy -2.754344 -2.750157)
    (xy -2.669824 -2.735552) (xy -2.568278 -2.702286) (xy -2.45567 -2.652661) (xy -2.337958 -2.588981) (xy -2.221105 -2.513547)
    (xy -2.112476 -2.429854) (xy -2.016667 -2.349429) (xy -1.946716 -2.294081) (xy -1.895715 -2.260626) (xy -1.856755 -2.245881)
    (xy -1.822927 -2.246663) (xy -1.787322 -2.259788) (xy -1.766134 -2.27027) (xy -1.701925 -2.295436) (xy -1.614888 -2.320084)
    (xy -1.53435 -2.336925) (xy -1.448012 -2.346938) (xy -1.342936 -2.352421) (xy -1.230517 -2.353563) (xy -1.122148 -2.350554)
    (xy -1.029226 -2.343585) (xy -0.963144 -2.332844) (xy -0.945835 -2.327121) (xy -0.911863 -2.325034) (xy -0.872043 -2.352958)
    (xy -0.844443 -2.382717) (xy -0.79818 -2.436499) (xy -0.736912 -2.507834) (xy -0.673788 -2.581415) (xy -0.672914 -2.582434)
    (xy -0.574448 -2.687746) (xy -0.469177 -2.783924) (xy -0.362999 -2.867111) (xy -0.261812 -2.933447) (xy -0.171515 -2.979075)
    (xy -0.098006 -3.000138))
   (stroke (width 0) (type solid)) (fill yes) (layer "F.Cu")))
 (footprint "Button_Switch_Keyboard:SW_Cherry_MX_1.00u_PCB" (layer "F.Cu") (at 147.499 79.2405)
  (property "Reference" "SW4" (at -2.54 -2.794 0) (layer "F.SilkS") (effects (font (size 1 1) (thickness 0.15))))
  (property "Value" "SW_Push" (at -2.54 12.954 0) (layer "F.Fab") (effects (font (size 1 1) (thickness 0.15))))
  (pad "" np_thru_hole circle (at -7.62 5.08) (size 1.7 1.7) (drill 1.7) (layers "*.Cu" "*.Mask"))
  (pad "" np_thru_hole circle (at -2.54 5.08) (size 4 4) (drill 4) (layers "*.Cu" "*.Mask"))
  (pad "" np_thru_hole circle (at 2.54 5.08) (size 1.7 1.7) (drill 1.7) (layers "*.Cu" "*.Mask"))
  (pad "1" thru_hole circle (at 0 0) (size 2.2 2.2) (drill 1.5) (layers "*.Cu" "*.Mask") (remove_unused_layers no) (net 9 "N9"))
  (pad "2" thru_hole circle (at -6.35 2.54) (size 2.2 2.2) (drill 1.5) (layers "*.Cu" "*.Mask") (remove_unused_layers no) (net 2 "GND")))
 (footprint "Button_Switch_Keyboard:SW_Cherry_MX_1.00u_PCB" (layer "F.Cu") (at 166.589 60.1505)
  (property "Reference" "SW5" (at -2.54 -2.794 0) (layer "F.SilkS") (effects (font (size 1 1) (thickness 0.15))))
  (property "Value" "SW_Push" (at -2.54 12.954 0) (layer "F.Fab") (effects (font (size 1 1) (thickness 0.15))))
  (pad "" np_thru_hole circle (at -7.62 5.08) (size 1.7 1.7) (drill 1.7) (layers "*.Cu" "*.Mask"))
  (pad "" np_thru_hole circle (at -2.54 5.08) (size 4 4) (drill 4) (layers "*.Cu" "*.Mask"))
  (pad "" np_thru_hole circle (at 2.54 5.08) (size 1.7 1.7) (drill 1.7) (layers "*.Cu" "*.Mask"))
  (pad "1" thru_hole circle (at 0 0) (size 2.2 2.2) (drill 1.5) (layers "*.Cu" "*.Mask") (remove_unused_layers no) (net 3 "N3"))
  (pad "2" thru_hole circle (at -6.35 2.54) (size 2.2 2.2) (drill 1.5) (layers "*.Cu" "*.Mask") (remove_unused_layers no) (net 2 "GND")))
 (gr_rect (start 116.19 21.4265) (end 173.725 93.9985) (stroke (width 0.05) (type default)) (fill no) (layer "Edge.Cuts"))
 (segment (start 141.149 81.7805) (end 122.059 81.7805) (width 0.2) (layer "F.Cu") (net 2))
 (segment (start 152.935 24.815) (end 152.935 25.62) (width 0.2) (layer "F.Cu") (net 2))
 (segment (start 159.572 55.155626) (end 159.833374 55.417) (width 0.2) (layer "F.Cu") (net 2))
 (segment (start 155.955 28.64) (end 154.654 27.339) (width 0.2) (layer "F.Cu") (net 2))
 (segment (start 154.654 24.839) (end 154.654 27.441) (width 0.2) (layer "F.Cu") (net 2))
 (segment (start 152.935 25.62) (end 155.955 28.64) (width 0.2) (layer "F.Cu") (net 2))
 (segment (start 141.149 62.6905) (end 122.059 62.6905) (width 0.2) (layer "F.Cu") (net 2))
 (segment (start 159.572 32.359) (end 159.572 55.155626) (width 0.2) (layer "F.Cu") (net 2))
 (segment (start 164.154 24.839) (end 154.654 24.839) (width 0.2) (layer "F.Cu") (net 2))
 (segment (start 160.239 62.6905) (end 168.255 54.6745) (width 0.2) (layer "F.Cu") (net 2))
 (segment (start 159.833374 55.417) (end 166.98063 55.417) (width 0.2) (layer "F.Cu") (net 2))
 (segment (start 122.059 62.6905) (end 122.059 81.7805) (width 0.2) (layer "F.Cu") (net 2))
 (segment (start 160.239 62.6905) (end 141.149 62.6905) (width 0.2) (layer "F.Cu") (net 2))
 (segment (start 168.255 54.6745) (end 168.255 53.065) (width 0.2) (layer "F.Cu") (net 2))
 (segment (start 166.98063 55.417) (end 168.255 54.14263) (width 0.2) (layer "F.Cu") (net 2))
 (segment (start 154.654 27.441) (end 159.572 32.359) (width 0.2) (layer "F.Cu") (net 2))
 (segment (start 170.455 31.14) (end 164.154 24.839) (width 0.2) (layer "F.Cu") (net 2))
 (segment (start 154.654 27.339) (end 154.654 24.839) (width 0.2) (layer "F.Cu") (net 2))
 (segment (start 160.239 81.7805) (end 141.149 81.7805) (width 0.2) (layer "F.Cu") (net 2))
 (segment (start 168.255 54.14263) (end 168.255 53.065) (width 0.2) (layer "F.Cu") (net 2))
 (via (at 153.575 24.2) (size 0.6) (drill 0.3) (layers "F.Cu" "B.Cu") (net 2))
 (segment (start 152.935 27.355) (end 151.784 28.506) (width 0.2) (layer "F.Cu") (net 13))
 (segment (start 165.715 53.065) (end 165.715 54.14263) (width 0.2) (layer "F.Cu") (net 13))
 (segment (start 151.784 28.506) (end 151.784 40.414) (width 0.2) (layer "F.Cu") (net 13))
 (segment (start 151.784 40.414) (end 156.155 44.785) (width 0.2) (layer "F.Cu") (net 13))
 (via (at 156.155 44.785) (size 0.6) (drill 0.3) (layers "F.Cu" "B.Cu") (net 13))
 (segment (start 156.446 44.494) (end 158.273943 44.494) (width 0.2) (layer "B.Cu") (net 13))
 (segment (start 158.273943 44.494) (end 165.715 51.935057) (width 0.2) (layer "B.Cu") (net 13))
 (segment (start 165.715 51.935057) (end 165.715 53.065) (width 0.2) (layer "B.Cu") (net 13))
 (segment (start 156.155 44.785) (end 156.446 44.494) (width 0.2) (layer "B.Cu") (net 13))
 (segment (start 169.318 43.968) (end 169.318 55.155626) (width 0.2) (layer "F.Cu") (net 5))
 (segment (start 163.175 37.825) (end 169.318 43.968) (width 0.2) (layer "F.Cu") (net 5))
 (segment (start 164.498626 59.975) (end 164.1 59.975) (width 0.2) (layer "F.Cu") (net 5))
 (segment (start 169.318 55.155626) (end 164.498626 59.975) (width 0.2) (layer "F.Cu") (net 5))
 (via (at 164.1 59.975) (size 0.6) (drill 0.3) (layers "F.Cu" "B.Cu") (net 5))
 (segment (start 156.618 52.62469) (end 154.44231 50.449) (width 0.2) (layer "B.Cu") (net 5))
 (segment (start 138.1105 50.449) (end 128.409 60.1505) (width 0.2) (layer "B.Cu") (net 5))
 (segment (start 154.44231 50.449) (end 138.1105 50.449) (width 0.2) (layer "B.Cu") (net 5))
 (segment (start 156.618 53.50531) (end 156.618 52.62469) (width 0.2) (layer "B.Cu") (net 5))
 (segment (start 164.1 59.975) (end 163.08769 59.975) (width 0.2) (layer "B.Cu") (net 5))
 (segment (start 163.08769 59.975) (end 156.618 53.50531) (width 0.2) (layer "B.Cu") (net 5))
 (segment (start 155.575 48.65) (end 153.175 51.05) (width 0.2) (layer "F.Cu") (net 8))
 (segment (start 155.575 46.75) (end 155.575 48.65) (width 0.2) (layer "F.Cu") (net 8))
 (via (at 155.575 46.75) (size 0.6) (drill 0.3) (layers "F.Cu" "B.Cu") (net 8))
 (via (at 153.175 51.05) (size 0.6) (drill 0.3) (layers "F.Cu" "B.Cu") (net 8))
 (segment (start 148.079314 58.7495) (end 146.918686 58.7495) (width 0.2) (layer "B.Cu") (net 8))
 (segment (start 155.555 37.825) (end 155.555 46.73) (width 0.2) (layer "B.Cu") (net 8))
 (segment (start 142.55 63.118186) (end 142.55 65.0995) (width 0.2) (layer "B.Cu") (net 8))
 (segment (start 153.175 53.653814) (end 148.079314 58.7495) (width 0.2) (layer "B.Cu") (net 8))
 (segment (start 146.918686 58.7495) (end 142.55 63.118186) (width 0.2) (layer "B.Cu") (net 8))
 (segment (start 155.555 46.73) (end 155.575 46.75) (width 0.2) (layer "B.Cu") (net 8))
 (segment (start 153.175 51.05) (end 153.175 53.653814) (width 0.2) (layer "B.Cu") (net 8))
 (segment (start 142.55 65.0995) (end 128.409 79.2405) (width 0.2) (layer "B.Cu") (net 8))
 (segment (start 165.715 37.825) (end 169.719 41.829) (width 0.2) (layer "F.Cu") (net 4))
 (segment (start 156.4495 60.1505) (end 147.499 60.1505) (width 0.2) (layer "F.Cu") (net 4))
 (segment (start 169.719 41.829) (end 169.719 59.001814) (width 0.2) (layer "F.Cu") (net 4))
 (segment (start 156.7 59.9) (end 156.4495 60.1505) (width 0.2) (layer "F.Cu") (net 4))
 (segment (start 169.719 59.001814) (end 166.720814 62) (width 0.2) (layer "F.Cu") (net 4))
 (segment (start 166.720814 62) (end 162.625 62) (width 0.2) (layer "F.Cu") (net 4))
 (via (at 162.625 62) (size 0.6) (drill 0.3) (layers "F.Cu" "B.Cu") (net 4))
 (via (at 156.7 59.9) (size 0.6) (drill 0.3) (layers "F.Cu" "B.Cu") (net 4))
 (segment (start 160.525 59.9) (end 156.7 59.9) (width 0.2) (layer "B.Cu") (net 4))
 (segment (start 162.625 62) (end 160.525 59.9) (width 0.2) (layer "B.Cu") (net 4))
 (segment (start 155.555 53.065) (end 155.555 71.1845) (width 0.2) (layer "B.Cu") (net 9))
 (segment (start 155.555 71.1845) (end 147.499 79.2405) (width 0.2) (layer "B.Cu") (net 9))
 (segment (start 172.65 39.68) (end 172.65 59.475) (width 0.2) (layer "F.Cu") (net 3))
 (segment (start 170.795 37.825) (end 172.65 39.68) (width 0.2) (layer "F.Cu") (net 3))
 (via (at 172.65 59.475) (size 0.6) (drill 0.3) (layers "F.Cu" "B.Cu") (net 3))
 (segment (start 172.65 59.475) (end 172.2 59.475) (width 0.2) (layer "B.Cu") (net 3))
 (segment (start 171.5245 60.1505) (end 166.589 60.1505) (width 0.2) (layer "B.Cu") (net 3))
 (segment (start 172.2 59.475) (end 171.5245 60.1505) (width 0.2) (layer "B.Cu") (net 3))
 (segment (start 168.255 37.825) (end 171.858 41.428) (width 0.2) (layer "F.Cu") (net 1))
 (segment (start 171.858 41.428) (end 171.858 73.9715) (width 0.2) (layer "F.Cu") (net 1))
 (segment (start 171.858 73.9715) (end 166.589 79.2405) (width 0.2) (layer "F.Cu") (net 1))
 (segment (start 162.112 36.099) (end 162.112 51.588) (width 0.2) (layer "F.Cu") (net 11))
 (segment (start 161.554 35.541) (end 162.112 36.099) (width 0.2) (layer "F.Cu") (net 11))
 (segment (start 162.112 51.588) (end 160.635 53.065) (width 0.2) (layer "F.Cu") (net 11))
 (segment (start 155.955 26.14) (end 161.554 31.739) (width 0.2) (layer "F.Cu") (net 11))
 (segment (start 161.554 31.739) (end 161.554 35.541) (width 0.2) (layer "F.Cu") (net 11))
 (segment (start 154.492 41.562) (end 158.025 45.095) (width 0.2) (layer "F.Cu") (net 12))
 (segment (start 155.955 31.14) (end 154.492 32.603) (width 0.2) (layer "F.Cu") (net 12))
 (segment (start 154.492 32.603) (end 154.492 41.562) (width 0.2) (layer "F.Cu") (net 12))
 (via (at 158.025 45.095) (size 0.6) (drill 0.3) (layers "F.Cu" "B.Cu") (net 12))
 (segment (start 158.025 45.095) (end 163.175 50.245) (width 0.2) (layer "B.Cu") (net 12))
 (segment (start 163.175 50.245) (end 163.175 53.065) (width 0.2) (layer "B.Cu") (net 12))
 (segment (start 158.856999 39.831999) (end 158.825 39.8) (width 0.2) (layer "F.Cu") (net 10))
 (segment (start 158.095 53.065) (end 158.856999 52.303001) (width 0.2) (layer "F.Cu") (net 10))
 (segment (start 158.856999 52.303001) (end 158.856999 39.831999) (width 0.2) (layer "F.Cu") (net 10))
 (via (at 158.825 39.8) (size 0.6) (drill 0.3) (layers "F.Cu" "B.Cu") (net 10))
 (segment (start 160.16331 39.8) (end 161.705 38.25831) (width 0.2) (layer "B.Cu") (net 10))
 (segment (start 158.825 39.8) (end 160.16331 39.8) (width 0.2) (layer "B.Cu") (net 10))
 (segment (start 161.705 35.692) (end 161.554 35.541) (width 0.2) (layer "B.Cu") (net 10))
 (segment (start 161.705 38.25831) (end 161.705 35.692) (width 0.2) (layer "B.Cu") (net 10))
 (segment (start 168.353 26.14) (end 170.455 26.14) (width 0.2) (layer "B.Cu") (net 10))
 (segment (start 161.554 32.939) (end 168.353 26.14) (width 0.2) (layer "B.Cu") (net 10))
 (segment (start 161.554 35.541) (end 161.554 32.939) (width 0.2) (layer "B.Cu") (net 10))
 (segment (start 154.086 34.339) (end 153.71 34.715) (width 0.2) (layer "F.Cu") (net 7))
 (segment (start 152.935 29.895) (end 154.086 31.046) (width 0.2) (layer "F.Cu") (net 7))
 (segment (start 154.086 31.046) (end 154.086 34.339) (width 0.2) (layer "F.Cu") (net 7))
 (via (at 153.71 34.715) (size 0.6) (drill 0.3) (layers "F.Cu" "B.Cu") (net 7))
 (segment (start 153.71 34.715) (end 154.985 34.715) (width 0.2) (layer "B.Cu") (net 7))
 (segment (start 154.985 34.715) (end 158.095 37.825) (width 0.2) (layer "B.Cu") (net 7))
 (segment (start 153.832 38.03) (end 153.892 38.09) (width 0.2) (layer "F.Cu") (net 6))
 (segment (start 153.46 38.03) (end 153.832 38.03) (width 0.2) (layer "F.Cu") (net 6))
 (segment (start 152.935 32.435) (end 152.935 37.505) (width 0.2) (layer "F.Cu") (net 6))
 (segment (start 152.935 37.505) (end 153.46 38.03) (width 0.2) (layer "F.Cu") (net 6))
 (via (at 153.892 38.09) (size 0.6) (drill 0.3) (layers "F.Cu" "B.Cu") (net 6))
 (segment (start 155.41169 36.465) (end 155.782 36.465) (width 0.2) (layer "B.Cu") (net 6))
 (segment (start 157.032 38.26531) (end 157.65469 38.888) (width 0.2) (layer "B.Cu") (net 6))
 (segment (start 157.65469 38.888) (end 159.572 38.888) (width 0.2) (layer "B.Cu") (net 6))
 (segment (start 153.892 38.09) (end 153.892 37.98469) (width 0.2) (layer "B.Cu") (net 6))
 (segment (start 159.572 38.888) (end 160.635 37.825) (width 0.2) (layer "B.Cu") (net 6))
 (segment (start 157.032 37.715) (end 157.032 38.26531) (width 0.2) (layer "B.Cu") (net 6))
 (segment (start 153.892 37.98469) (end 155.41169 36.465) (width 0.2) (layer "B.Cu") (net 6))
 (segment (start 155.782 36.465) (end 157.032 37.715) (width 0.2) (layer "B.Cu") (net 6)))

